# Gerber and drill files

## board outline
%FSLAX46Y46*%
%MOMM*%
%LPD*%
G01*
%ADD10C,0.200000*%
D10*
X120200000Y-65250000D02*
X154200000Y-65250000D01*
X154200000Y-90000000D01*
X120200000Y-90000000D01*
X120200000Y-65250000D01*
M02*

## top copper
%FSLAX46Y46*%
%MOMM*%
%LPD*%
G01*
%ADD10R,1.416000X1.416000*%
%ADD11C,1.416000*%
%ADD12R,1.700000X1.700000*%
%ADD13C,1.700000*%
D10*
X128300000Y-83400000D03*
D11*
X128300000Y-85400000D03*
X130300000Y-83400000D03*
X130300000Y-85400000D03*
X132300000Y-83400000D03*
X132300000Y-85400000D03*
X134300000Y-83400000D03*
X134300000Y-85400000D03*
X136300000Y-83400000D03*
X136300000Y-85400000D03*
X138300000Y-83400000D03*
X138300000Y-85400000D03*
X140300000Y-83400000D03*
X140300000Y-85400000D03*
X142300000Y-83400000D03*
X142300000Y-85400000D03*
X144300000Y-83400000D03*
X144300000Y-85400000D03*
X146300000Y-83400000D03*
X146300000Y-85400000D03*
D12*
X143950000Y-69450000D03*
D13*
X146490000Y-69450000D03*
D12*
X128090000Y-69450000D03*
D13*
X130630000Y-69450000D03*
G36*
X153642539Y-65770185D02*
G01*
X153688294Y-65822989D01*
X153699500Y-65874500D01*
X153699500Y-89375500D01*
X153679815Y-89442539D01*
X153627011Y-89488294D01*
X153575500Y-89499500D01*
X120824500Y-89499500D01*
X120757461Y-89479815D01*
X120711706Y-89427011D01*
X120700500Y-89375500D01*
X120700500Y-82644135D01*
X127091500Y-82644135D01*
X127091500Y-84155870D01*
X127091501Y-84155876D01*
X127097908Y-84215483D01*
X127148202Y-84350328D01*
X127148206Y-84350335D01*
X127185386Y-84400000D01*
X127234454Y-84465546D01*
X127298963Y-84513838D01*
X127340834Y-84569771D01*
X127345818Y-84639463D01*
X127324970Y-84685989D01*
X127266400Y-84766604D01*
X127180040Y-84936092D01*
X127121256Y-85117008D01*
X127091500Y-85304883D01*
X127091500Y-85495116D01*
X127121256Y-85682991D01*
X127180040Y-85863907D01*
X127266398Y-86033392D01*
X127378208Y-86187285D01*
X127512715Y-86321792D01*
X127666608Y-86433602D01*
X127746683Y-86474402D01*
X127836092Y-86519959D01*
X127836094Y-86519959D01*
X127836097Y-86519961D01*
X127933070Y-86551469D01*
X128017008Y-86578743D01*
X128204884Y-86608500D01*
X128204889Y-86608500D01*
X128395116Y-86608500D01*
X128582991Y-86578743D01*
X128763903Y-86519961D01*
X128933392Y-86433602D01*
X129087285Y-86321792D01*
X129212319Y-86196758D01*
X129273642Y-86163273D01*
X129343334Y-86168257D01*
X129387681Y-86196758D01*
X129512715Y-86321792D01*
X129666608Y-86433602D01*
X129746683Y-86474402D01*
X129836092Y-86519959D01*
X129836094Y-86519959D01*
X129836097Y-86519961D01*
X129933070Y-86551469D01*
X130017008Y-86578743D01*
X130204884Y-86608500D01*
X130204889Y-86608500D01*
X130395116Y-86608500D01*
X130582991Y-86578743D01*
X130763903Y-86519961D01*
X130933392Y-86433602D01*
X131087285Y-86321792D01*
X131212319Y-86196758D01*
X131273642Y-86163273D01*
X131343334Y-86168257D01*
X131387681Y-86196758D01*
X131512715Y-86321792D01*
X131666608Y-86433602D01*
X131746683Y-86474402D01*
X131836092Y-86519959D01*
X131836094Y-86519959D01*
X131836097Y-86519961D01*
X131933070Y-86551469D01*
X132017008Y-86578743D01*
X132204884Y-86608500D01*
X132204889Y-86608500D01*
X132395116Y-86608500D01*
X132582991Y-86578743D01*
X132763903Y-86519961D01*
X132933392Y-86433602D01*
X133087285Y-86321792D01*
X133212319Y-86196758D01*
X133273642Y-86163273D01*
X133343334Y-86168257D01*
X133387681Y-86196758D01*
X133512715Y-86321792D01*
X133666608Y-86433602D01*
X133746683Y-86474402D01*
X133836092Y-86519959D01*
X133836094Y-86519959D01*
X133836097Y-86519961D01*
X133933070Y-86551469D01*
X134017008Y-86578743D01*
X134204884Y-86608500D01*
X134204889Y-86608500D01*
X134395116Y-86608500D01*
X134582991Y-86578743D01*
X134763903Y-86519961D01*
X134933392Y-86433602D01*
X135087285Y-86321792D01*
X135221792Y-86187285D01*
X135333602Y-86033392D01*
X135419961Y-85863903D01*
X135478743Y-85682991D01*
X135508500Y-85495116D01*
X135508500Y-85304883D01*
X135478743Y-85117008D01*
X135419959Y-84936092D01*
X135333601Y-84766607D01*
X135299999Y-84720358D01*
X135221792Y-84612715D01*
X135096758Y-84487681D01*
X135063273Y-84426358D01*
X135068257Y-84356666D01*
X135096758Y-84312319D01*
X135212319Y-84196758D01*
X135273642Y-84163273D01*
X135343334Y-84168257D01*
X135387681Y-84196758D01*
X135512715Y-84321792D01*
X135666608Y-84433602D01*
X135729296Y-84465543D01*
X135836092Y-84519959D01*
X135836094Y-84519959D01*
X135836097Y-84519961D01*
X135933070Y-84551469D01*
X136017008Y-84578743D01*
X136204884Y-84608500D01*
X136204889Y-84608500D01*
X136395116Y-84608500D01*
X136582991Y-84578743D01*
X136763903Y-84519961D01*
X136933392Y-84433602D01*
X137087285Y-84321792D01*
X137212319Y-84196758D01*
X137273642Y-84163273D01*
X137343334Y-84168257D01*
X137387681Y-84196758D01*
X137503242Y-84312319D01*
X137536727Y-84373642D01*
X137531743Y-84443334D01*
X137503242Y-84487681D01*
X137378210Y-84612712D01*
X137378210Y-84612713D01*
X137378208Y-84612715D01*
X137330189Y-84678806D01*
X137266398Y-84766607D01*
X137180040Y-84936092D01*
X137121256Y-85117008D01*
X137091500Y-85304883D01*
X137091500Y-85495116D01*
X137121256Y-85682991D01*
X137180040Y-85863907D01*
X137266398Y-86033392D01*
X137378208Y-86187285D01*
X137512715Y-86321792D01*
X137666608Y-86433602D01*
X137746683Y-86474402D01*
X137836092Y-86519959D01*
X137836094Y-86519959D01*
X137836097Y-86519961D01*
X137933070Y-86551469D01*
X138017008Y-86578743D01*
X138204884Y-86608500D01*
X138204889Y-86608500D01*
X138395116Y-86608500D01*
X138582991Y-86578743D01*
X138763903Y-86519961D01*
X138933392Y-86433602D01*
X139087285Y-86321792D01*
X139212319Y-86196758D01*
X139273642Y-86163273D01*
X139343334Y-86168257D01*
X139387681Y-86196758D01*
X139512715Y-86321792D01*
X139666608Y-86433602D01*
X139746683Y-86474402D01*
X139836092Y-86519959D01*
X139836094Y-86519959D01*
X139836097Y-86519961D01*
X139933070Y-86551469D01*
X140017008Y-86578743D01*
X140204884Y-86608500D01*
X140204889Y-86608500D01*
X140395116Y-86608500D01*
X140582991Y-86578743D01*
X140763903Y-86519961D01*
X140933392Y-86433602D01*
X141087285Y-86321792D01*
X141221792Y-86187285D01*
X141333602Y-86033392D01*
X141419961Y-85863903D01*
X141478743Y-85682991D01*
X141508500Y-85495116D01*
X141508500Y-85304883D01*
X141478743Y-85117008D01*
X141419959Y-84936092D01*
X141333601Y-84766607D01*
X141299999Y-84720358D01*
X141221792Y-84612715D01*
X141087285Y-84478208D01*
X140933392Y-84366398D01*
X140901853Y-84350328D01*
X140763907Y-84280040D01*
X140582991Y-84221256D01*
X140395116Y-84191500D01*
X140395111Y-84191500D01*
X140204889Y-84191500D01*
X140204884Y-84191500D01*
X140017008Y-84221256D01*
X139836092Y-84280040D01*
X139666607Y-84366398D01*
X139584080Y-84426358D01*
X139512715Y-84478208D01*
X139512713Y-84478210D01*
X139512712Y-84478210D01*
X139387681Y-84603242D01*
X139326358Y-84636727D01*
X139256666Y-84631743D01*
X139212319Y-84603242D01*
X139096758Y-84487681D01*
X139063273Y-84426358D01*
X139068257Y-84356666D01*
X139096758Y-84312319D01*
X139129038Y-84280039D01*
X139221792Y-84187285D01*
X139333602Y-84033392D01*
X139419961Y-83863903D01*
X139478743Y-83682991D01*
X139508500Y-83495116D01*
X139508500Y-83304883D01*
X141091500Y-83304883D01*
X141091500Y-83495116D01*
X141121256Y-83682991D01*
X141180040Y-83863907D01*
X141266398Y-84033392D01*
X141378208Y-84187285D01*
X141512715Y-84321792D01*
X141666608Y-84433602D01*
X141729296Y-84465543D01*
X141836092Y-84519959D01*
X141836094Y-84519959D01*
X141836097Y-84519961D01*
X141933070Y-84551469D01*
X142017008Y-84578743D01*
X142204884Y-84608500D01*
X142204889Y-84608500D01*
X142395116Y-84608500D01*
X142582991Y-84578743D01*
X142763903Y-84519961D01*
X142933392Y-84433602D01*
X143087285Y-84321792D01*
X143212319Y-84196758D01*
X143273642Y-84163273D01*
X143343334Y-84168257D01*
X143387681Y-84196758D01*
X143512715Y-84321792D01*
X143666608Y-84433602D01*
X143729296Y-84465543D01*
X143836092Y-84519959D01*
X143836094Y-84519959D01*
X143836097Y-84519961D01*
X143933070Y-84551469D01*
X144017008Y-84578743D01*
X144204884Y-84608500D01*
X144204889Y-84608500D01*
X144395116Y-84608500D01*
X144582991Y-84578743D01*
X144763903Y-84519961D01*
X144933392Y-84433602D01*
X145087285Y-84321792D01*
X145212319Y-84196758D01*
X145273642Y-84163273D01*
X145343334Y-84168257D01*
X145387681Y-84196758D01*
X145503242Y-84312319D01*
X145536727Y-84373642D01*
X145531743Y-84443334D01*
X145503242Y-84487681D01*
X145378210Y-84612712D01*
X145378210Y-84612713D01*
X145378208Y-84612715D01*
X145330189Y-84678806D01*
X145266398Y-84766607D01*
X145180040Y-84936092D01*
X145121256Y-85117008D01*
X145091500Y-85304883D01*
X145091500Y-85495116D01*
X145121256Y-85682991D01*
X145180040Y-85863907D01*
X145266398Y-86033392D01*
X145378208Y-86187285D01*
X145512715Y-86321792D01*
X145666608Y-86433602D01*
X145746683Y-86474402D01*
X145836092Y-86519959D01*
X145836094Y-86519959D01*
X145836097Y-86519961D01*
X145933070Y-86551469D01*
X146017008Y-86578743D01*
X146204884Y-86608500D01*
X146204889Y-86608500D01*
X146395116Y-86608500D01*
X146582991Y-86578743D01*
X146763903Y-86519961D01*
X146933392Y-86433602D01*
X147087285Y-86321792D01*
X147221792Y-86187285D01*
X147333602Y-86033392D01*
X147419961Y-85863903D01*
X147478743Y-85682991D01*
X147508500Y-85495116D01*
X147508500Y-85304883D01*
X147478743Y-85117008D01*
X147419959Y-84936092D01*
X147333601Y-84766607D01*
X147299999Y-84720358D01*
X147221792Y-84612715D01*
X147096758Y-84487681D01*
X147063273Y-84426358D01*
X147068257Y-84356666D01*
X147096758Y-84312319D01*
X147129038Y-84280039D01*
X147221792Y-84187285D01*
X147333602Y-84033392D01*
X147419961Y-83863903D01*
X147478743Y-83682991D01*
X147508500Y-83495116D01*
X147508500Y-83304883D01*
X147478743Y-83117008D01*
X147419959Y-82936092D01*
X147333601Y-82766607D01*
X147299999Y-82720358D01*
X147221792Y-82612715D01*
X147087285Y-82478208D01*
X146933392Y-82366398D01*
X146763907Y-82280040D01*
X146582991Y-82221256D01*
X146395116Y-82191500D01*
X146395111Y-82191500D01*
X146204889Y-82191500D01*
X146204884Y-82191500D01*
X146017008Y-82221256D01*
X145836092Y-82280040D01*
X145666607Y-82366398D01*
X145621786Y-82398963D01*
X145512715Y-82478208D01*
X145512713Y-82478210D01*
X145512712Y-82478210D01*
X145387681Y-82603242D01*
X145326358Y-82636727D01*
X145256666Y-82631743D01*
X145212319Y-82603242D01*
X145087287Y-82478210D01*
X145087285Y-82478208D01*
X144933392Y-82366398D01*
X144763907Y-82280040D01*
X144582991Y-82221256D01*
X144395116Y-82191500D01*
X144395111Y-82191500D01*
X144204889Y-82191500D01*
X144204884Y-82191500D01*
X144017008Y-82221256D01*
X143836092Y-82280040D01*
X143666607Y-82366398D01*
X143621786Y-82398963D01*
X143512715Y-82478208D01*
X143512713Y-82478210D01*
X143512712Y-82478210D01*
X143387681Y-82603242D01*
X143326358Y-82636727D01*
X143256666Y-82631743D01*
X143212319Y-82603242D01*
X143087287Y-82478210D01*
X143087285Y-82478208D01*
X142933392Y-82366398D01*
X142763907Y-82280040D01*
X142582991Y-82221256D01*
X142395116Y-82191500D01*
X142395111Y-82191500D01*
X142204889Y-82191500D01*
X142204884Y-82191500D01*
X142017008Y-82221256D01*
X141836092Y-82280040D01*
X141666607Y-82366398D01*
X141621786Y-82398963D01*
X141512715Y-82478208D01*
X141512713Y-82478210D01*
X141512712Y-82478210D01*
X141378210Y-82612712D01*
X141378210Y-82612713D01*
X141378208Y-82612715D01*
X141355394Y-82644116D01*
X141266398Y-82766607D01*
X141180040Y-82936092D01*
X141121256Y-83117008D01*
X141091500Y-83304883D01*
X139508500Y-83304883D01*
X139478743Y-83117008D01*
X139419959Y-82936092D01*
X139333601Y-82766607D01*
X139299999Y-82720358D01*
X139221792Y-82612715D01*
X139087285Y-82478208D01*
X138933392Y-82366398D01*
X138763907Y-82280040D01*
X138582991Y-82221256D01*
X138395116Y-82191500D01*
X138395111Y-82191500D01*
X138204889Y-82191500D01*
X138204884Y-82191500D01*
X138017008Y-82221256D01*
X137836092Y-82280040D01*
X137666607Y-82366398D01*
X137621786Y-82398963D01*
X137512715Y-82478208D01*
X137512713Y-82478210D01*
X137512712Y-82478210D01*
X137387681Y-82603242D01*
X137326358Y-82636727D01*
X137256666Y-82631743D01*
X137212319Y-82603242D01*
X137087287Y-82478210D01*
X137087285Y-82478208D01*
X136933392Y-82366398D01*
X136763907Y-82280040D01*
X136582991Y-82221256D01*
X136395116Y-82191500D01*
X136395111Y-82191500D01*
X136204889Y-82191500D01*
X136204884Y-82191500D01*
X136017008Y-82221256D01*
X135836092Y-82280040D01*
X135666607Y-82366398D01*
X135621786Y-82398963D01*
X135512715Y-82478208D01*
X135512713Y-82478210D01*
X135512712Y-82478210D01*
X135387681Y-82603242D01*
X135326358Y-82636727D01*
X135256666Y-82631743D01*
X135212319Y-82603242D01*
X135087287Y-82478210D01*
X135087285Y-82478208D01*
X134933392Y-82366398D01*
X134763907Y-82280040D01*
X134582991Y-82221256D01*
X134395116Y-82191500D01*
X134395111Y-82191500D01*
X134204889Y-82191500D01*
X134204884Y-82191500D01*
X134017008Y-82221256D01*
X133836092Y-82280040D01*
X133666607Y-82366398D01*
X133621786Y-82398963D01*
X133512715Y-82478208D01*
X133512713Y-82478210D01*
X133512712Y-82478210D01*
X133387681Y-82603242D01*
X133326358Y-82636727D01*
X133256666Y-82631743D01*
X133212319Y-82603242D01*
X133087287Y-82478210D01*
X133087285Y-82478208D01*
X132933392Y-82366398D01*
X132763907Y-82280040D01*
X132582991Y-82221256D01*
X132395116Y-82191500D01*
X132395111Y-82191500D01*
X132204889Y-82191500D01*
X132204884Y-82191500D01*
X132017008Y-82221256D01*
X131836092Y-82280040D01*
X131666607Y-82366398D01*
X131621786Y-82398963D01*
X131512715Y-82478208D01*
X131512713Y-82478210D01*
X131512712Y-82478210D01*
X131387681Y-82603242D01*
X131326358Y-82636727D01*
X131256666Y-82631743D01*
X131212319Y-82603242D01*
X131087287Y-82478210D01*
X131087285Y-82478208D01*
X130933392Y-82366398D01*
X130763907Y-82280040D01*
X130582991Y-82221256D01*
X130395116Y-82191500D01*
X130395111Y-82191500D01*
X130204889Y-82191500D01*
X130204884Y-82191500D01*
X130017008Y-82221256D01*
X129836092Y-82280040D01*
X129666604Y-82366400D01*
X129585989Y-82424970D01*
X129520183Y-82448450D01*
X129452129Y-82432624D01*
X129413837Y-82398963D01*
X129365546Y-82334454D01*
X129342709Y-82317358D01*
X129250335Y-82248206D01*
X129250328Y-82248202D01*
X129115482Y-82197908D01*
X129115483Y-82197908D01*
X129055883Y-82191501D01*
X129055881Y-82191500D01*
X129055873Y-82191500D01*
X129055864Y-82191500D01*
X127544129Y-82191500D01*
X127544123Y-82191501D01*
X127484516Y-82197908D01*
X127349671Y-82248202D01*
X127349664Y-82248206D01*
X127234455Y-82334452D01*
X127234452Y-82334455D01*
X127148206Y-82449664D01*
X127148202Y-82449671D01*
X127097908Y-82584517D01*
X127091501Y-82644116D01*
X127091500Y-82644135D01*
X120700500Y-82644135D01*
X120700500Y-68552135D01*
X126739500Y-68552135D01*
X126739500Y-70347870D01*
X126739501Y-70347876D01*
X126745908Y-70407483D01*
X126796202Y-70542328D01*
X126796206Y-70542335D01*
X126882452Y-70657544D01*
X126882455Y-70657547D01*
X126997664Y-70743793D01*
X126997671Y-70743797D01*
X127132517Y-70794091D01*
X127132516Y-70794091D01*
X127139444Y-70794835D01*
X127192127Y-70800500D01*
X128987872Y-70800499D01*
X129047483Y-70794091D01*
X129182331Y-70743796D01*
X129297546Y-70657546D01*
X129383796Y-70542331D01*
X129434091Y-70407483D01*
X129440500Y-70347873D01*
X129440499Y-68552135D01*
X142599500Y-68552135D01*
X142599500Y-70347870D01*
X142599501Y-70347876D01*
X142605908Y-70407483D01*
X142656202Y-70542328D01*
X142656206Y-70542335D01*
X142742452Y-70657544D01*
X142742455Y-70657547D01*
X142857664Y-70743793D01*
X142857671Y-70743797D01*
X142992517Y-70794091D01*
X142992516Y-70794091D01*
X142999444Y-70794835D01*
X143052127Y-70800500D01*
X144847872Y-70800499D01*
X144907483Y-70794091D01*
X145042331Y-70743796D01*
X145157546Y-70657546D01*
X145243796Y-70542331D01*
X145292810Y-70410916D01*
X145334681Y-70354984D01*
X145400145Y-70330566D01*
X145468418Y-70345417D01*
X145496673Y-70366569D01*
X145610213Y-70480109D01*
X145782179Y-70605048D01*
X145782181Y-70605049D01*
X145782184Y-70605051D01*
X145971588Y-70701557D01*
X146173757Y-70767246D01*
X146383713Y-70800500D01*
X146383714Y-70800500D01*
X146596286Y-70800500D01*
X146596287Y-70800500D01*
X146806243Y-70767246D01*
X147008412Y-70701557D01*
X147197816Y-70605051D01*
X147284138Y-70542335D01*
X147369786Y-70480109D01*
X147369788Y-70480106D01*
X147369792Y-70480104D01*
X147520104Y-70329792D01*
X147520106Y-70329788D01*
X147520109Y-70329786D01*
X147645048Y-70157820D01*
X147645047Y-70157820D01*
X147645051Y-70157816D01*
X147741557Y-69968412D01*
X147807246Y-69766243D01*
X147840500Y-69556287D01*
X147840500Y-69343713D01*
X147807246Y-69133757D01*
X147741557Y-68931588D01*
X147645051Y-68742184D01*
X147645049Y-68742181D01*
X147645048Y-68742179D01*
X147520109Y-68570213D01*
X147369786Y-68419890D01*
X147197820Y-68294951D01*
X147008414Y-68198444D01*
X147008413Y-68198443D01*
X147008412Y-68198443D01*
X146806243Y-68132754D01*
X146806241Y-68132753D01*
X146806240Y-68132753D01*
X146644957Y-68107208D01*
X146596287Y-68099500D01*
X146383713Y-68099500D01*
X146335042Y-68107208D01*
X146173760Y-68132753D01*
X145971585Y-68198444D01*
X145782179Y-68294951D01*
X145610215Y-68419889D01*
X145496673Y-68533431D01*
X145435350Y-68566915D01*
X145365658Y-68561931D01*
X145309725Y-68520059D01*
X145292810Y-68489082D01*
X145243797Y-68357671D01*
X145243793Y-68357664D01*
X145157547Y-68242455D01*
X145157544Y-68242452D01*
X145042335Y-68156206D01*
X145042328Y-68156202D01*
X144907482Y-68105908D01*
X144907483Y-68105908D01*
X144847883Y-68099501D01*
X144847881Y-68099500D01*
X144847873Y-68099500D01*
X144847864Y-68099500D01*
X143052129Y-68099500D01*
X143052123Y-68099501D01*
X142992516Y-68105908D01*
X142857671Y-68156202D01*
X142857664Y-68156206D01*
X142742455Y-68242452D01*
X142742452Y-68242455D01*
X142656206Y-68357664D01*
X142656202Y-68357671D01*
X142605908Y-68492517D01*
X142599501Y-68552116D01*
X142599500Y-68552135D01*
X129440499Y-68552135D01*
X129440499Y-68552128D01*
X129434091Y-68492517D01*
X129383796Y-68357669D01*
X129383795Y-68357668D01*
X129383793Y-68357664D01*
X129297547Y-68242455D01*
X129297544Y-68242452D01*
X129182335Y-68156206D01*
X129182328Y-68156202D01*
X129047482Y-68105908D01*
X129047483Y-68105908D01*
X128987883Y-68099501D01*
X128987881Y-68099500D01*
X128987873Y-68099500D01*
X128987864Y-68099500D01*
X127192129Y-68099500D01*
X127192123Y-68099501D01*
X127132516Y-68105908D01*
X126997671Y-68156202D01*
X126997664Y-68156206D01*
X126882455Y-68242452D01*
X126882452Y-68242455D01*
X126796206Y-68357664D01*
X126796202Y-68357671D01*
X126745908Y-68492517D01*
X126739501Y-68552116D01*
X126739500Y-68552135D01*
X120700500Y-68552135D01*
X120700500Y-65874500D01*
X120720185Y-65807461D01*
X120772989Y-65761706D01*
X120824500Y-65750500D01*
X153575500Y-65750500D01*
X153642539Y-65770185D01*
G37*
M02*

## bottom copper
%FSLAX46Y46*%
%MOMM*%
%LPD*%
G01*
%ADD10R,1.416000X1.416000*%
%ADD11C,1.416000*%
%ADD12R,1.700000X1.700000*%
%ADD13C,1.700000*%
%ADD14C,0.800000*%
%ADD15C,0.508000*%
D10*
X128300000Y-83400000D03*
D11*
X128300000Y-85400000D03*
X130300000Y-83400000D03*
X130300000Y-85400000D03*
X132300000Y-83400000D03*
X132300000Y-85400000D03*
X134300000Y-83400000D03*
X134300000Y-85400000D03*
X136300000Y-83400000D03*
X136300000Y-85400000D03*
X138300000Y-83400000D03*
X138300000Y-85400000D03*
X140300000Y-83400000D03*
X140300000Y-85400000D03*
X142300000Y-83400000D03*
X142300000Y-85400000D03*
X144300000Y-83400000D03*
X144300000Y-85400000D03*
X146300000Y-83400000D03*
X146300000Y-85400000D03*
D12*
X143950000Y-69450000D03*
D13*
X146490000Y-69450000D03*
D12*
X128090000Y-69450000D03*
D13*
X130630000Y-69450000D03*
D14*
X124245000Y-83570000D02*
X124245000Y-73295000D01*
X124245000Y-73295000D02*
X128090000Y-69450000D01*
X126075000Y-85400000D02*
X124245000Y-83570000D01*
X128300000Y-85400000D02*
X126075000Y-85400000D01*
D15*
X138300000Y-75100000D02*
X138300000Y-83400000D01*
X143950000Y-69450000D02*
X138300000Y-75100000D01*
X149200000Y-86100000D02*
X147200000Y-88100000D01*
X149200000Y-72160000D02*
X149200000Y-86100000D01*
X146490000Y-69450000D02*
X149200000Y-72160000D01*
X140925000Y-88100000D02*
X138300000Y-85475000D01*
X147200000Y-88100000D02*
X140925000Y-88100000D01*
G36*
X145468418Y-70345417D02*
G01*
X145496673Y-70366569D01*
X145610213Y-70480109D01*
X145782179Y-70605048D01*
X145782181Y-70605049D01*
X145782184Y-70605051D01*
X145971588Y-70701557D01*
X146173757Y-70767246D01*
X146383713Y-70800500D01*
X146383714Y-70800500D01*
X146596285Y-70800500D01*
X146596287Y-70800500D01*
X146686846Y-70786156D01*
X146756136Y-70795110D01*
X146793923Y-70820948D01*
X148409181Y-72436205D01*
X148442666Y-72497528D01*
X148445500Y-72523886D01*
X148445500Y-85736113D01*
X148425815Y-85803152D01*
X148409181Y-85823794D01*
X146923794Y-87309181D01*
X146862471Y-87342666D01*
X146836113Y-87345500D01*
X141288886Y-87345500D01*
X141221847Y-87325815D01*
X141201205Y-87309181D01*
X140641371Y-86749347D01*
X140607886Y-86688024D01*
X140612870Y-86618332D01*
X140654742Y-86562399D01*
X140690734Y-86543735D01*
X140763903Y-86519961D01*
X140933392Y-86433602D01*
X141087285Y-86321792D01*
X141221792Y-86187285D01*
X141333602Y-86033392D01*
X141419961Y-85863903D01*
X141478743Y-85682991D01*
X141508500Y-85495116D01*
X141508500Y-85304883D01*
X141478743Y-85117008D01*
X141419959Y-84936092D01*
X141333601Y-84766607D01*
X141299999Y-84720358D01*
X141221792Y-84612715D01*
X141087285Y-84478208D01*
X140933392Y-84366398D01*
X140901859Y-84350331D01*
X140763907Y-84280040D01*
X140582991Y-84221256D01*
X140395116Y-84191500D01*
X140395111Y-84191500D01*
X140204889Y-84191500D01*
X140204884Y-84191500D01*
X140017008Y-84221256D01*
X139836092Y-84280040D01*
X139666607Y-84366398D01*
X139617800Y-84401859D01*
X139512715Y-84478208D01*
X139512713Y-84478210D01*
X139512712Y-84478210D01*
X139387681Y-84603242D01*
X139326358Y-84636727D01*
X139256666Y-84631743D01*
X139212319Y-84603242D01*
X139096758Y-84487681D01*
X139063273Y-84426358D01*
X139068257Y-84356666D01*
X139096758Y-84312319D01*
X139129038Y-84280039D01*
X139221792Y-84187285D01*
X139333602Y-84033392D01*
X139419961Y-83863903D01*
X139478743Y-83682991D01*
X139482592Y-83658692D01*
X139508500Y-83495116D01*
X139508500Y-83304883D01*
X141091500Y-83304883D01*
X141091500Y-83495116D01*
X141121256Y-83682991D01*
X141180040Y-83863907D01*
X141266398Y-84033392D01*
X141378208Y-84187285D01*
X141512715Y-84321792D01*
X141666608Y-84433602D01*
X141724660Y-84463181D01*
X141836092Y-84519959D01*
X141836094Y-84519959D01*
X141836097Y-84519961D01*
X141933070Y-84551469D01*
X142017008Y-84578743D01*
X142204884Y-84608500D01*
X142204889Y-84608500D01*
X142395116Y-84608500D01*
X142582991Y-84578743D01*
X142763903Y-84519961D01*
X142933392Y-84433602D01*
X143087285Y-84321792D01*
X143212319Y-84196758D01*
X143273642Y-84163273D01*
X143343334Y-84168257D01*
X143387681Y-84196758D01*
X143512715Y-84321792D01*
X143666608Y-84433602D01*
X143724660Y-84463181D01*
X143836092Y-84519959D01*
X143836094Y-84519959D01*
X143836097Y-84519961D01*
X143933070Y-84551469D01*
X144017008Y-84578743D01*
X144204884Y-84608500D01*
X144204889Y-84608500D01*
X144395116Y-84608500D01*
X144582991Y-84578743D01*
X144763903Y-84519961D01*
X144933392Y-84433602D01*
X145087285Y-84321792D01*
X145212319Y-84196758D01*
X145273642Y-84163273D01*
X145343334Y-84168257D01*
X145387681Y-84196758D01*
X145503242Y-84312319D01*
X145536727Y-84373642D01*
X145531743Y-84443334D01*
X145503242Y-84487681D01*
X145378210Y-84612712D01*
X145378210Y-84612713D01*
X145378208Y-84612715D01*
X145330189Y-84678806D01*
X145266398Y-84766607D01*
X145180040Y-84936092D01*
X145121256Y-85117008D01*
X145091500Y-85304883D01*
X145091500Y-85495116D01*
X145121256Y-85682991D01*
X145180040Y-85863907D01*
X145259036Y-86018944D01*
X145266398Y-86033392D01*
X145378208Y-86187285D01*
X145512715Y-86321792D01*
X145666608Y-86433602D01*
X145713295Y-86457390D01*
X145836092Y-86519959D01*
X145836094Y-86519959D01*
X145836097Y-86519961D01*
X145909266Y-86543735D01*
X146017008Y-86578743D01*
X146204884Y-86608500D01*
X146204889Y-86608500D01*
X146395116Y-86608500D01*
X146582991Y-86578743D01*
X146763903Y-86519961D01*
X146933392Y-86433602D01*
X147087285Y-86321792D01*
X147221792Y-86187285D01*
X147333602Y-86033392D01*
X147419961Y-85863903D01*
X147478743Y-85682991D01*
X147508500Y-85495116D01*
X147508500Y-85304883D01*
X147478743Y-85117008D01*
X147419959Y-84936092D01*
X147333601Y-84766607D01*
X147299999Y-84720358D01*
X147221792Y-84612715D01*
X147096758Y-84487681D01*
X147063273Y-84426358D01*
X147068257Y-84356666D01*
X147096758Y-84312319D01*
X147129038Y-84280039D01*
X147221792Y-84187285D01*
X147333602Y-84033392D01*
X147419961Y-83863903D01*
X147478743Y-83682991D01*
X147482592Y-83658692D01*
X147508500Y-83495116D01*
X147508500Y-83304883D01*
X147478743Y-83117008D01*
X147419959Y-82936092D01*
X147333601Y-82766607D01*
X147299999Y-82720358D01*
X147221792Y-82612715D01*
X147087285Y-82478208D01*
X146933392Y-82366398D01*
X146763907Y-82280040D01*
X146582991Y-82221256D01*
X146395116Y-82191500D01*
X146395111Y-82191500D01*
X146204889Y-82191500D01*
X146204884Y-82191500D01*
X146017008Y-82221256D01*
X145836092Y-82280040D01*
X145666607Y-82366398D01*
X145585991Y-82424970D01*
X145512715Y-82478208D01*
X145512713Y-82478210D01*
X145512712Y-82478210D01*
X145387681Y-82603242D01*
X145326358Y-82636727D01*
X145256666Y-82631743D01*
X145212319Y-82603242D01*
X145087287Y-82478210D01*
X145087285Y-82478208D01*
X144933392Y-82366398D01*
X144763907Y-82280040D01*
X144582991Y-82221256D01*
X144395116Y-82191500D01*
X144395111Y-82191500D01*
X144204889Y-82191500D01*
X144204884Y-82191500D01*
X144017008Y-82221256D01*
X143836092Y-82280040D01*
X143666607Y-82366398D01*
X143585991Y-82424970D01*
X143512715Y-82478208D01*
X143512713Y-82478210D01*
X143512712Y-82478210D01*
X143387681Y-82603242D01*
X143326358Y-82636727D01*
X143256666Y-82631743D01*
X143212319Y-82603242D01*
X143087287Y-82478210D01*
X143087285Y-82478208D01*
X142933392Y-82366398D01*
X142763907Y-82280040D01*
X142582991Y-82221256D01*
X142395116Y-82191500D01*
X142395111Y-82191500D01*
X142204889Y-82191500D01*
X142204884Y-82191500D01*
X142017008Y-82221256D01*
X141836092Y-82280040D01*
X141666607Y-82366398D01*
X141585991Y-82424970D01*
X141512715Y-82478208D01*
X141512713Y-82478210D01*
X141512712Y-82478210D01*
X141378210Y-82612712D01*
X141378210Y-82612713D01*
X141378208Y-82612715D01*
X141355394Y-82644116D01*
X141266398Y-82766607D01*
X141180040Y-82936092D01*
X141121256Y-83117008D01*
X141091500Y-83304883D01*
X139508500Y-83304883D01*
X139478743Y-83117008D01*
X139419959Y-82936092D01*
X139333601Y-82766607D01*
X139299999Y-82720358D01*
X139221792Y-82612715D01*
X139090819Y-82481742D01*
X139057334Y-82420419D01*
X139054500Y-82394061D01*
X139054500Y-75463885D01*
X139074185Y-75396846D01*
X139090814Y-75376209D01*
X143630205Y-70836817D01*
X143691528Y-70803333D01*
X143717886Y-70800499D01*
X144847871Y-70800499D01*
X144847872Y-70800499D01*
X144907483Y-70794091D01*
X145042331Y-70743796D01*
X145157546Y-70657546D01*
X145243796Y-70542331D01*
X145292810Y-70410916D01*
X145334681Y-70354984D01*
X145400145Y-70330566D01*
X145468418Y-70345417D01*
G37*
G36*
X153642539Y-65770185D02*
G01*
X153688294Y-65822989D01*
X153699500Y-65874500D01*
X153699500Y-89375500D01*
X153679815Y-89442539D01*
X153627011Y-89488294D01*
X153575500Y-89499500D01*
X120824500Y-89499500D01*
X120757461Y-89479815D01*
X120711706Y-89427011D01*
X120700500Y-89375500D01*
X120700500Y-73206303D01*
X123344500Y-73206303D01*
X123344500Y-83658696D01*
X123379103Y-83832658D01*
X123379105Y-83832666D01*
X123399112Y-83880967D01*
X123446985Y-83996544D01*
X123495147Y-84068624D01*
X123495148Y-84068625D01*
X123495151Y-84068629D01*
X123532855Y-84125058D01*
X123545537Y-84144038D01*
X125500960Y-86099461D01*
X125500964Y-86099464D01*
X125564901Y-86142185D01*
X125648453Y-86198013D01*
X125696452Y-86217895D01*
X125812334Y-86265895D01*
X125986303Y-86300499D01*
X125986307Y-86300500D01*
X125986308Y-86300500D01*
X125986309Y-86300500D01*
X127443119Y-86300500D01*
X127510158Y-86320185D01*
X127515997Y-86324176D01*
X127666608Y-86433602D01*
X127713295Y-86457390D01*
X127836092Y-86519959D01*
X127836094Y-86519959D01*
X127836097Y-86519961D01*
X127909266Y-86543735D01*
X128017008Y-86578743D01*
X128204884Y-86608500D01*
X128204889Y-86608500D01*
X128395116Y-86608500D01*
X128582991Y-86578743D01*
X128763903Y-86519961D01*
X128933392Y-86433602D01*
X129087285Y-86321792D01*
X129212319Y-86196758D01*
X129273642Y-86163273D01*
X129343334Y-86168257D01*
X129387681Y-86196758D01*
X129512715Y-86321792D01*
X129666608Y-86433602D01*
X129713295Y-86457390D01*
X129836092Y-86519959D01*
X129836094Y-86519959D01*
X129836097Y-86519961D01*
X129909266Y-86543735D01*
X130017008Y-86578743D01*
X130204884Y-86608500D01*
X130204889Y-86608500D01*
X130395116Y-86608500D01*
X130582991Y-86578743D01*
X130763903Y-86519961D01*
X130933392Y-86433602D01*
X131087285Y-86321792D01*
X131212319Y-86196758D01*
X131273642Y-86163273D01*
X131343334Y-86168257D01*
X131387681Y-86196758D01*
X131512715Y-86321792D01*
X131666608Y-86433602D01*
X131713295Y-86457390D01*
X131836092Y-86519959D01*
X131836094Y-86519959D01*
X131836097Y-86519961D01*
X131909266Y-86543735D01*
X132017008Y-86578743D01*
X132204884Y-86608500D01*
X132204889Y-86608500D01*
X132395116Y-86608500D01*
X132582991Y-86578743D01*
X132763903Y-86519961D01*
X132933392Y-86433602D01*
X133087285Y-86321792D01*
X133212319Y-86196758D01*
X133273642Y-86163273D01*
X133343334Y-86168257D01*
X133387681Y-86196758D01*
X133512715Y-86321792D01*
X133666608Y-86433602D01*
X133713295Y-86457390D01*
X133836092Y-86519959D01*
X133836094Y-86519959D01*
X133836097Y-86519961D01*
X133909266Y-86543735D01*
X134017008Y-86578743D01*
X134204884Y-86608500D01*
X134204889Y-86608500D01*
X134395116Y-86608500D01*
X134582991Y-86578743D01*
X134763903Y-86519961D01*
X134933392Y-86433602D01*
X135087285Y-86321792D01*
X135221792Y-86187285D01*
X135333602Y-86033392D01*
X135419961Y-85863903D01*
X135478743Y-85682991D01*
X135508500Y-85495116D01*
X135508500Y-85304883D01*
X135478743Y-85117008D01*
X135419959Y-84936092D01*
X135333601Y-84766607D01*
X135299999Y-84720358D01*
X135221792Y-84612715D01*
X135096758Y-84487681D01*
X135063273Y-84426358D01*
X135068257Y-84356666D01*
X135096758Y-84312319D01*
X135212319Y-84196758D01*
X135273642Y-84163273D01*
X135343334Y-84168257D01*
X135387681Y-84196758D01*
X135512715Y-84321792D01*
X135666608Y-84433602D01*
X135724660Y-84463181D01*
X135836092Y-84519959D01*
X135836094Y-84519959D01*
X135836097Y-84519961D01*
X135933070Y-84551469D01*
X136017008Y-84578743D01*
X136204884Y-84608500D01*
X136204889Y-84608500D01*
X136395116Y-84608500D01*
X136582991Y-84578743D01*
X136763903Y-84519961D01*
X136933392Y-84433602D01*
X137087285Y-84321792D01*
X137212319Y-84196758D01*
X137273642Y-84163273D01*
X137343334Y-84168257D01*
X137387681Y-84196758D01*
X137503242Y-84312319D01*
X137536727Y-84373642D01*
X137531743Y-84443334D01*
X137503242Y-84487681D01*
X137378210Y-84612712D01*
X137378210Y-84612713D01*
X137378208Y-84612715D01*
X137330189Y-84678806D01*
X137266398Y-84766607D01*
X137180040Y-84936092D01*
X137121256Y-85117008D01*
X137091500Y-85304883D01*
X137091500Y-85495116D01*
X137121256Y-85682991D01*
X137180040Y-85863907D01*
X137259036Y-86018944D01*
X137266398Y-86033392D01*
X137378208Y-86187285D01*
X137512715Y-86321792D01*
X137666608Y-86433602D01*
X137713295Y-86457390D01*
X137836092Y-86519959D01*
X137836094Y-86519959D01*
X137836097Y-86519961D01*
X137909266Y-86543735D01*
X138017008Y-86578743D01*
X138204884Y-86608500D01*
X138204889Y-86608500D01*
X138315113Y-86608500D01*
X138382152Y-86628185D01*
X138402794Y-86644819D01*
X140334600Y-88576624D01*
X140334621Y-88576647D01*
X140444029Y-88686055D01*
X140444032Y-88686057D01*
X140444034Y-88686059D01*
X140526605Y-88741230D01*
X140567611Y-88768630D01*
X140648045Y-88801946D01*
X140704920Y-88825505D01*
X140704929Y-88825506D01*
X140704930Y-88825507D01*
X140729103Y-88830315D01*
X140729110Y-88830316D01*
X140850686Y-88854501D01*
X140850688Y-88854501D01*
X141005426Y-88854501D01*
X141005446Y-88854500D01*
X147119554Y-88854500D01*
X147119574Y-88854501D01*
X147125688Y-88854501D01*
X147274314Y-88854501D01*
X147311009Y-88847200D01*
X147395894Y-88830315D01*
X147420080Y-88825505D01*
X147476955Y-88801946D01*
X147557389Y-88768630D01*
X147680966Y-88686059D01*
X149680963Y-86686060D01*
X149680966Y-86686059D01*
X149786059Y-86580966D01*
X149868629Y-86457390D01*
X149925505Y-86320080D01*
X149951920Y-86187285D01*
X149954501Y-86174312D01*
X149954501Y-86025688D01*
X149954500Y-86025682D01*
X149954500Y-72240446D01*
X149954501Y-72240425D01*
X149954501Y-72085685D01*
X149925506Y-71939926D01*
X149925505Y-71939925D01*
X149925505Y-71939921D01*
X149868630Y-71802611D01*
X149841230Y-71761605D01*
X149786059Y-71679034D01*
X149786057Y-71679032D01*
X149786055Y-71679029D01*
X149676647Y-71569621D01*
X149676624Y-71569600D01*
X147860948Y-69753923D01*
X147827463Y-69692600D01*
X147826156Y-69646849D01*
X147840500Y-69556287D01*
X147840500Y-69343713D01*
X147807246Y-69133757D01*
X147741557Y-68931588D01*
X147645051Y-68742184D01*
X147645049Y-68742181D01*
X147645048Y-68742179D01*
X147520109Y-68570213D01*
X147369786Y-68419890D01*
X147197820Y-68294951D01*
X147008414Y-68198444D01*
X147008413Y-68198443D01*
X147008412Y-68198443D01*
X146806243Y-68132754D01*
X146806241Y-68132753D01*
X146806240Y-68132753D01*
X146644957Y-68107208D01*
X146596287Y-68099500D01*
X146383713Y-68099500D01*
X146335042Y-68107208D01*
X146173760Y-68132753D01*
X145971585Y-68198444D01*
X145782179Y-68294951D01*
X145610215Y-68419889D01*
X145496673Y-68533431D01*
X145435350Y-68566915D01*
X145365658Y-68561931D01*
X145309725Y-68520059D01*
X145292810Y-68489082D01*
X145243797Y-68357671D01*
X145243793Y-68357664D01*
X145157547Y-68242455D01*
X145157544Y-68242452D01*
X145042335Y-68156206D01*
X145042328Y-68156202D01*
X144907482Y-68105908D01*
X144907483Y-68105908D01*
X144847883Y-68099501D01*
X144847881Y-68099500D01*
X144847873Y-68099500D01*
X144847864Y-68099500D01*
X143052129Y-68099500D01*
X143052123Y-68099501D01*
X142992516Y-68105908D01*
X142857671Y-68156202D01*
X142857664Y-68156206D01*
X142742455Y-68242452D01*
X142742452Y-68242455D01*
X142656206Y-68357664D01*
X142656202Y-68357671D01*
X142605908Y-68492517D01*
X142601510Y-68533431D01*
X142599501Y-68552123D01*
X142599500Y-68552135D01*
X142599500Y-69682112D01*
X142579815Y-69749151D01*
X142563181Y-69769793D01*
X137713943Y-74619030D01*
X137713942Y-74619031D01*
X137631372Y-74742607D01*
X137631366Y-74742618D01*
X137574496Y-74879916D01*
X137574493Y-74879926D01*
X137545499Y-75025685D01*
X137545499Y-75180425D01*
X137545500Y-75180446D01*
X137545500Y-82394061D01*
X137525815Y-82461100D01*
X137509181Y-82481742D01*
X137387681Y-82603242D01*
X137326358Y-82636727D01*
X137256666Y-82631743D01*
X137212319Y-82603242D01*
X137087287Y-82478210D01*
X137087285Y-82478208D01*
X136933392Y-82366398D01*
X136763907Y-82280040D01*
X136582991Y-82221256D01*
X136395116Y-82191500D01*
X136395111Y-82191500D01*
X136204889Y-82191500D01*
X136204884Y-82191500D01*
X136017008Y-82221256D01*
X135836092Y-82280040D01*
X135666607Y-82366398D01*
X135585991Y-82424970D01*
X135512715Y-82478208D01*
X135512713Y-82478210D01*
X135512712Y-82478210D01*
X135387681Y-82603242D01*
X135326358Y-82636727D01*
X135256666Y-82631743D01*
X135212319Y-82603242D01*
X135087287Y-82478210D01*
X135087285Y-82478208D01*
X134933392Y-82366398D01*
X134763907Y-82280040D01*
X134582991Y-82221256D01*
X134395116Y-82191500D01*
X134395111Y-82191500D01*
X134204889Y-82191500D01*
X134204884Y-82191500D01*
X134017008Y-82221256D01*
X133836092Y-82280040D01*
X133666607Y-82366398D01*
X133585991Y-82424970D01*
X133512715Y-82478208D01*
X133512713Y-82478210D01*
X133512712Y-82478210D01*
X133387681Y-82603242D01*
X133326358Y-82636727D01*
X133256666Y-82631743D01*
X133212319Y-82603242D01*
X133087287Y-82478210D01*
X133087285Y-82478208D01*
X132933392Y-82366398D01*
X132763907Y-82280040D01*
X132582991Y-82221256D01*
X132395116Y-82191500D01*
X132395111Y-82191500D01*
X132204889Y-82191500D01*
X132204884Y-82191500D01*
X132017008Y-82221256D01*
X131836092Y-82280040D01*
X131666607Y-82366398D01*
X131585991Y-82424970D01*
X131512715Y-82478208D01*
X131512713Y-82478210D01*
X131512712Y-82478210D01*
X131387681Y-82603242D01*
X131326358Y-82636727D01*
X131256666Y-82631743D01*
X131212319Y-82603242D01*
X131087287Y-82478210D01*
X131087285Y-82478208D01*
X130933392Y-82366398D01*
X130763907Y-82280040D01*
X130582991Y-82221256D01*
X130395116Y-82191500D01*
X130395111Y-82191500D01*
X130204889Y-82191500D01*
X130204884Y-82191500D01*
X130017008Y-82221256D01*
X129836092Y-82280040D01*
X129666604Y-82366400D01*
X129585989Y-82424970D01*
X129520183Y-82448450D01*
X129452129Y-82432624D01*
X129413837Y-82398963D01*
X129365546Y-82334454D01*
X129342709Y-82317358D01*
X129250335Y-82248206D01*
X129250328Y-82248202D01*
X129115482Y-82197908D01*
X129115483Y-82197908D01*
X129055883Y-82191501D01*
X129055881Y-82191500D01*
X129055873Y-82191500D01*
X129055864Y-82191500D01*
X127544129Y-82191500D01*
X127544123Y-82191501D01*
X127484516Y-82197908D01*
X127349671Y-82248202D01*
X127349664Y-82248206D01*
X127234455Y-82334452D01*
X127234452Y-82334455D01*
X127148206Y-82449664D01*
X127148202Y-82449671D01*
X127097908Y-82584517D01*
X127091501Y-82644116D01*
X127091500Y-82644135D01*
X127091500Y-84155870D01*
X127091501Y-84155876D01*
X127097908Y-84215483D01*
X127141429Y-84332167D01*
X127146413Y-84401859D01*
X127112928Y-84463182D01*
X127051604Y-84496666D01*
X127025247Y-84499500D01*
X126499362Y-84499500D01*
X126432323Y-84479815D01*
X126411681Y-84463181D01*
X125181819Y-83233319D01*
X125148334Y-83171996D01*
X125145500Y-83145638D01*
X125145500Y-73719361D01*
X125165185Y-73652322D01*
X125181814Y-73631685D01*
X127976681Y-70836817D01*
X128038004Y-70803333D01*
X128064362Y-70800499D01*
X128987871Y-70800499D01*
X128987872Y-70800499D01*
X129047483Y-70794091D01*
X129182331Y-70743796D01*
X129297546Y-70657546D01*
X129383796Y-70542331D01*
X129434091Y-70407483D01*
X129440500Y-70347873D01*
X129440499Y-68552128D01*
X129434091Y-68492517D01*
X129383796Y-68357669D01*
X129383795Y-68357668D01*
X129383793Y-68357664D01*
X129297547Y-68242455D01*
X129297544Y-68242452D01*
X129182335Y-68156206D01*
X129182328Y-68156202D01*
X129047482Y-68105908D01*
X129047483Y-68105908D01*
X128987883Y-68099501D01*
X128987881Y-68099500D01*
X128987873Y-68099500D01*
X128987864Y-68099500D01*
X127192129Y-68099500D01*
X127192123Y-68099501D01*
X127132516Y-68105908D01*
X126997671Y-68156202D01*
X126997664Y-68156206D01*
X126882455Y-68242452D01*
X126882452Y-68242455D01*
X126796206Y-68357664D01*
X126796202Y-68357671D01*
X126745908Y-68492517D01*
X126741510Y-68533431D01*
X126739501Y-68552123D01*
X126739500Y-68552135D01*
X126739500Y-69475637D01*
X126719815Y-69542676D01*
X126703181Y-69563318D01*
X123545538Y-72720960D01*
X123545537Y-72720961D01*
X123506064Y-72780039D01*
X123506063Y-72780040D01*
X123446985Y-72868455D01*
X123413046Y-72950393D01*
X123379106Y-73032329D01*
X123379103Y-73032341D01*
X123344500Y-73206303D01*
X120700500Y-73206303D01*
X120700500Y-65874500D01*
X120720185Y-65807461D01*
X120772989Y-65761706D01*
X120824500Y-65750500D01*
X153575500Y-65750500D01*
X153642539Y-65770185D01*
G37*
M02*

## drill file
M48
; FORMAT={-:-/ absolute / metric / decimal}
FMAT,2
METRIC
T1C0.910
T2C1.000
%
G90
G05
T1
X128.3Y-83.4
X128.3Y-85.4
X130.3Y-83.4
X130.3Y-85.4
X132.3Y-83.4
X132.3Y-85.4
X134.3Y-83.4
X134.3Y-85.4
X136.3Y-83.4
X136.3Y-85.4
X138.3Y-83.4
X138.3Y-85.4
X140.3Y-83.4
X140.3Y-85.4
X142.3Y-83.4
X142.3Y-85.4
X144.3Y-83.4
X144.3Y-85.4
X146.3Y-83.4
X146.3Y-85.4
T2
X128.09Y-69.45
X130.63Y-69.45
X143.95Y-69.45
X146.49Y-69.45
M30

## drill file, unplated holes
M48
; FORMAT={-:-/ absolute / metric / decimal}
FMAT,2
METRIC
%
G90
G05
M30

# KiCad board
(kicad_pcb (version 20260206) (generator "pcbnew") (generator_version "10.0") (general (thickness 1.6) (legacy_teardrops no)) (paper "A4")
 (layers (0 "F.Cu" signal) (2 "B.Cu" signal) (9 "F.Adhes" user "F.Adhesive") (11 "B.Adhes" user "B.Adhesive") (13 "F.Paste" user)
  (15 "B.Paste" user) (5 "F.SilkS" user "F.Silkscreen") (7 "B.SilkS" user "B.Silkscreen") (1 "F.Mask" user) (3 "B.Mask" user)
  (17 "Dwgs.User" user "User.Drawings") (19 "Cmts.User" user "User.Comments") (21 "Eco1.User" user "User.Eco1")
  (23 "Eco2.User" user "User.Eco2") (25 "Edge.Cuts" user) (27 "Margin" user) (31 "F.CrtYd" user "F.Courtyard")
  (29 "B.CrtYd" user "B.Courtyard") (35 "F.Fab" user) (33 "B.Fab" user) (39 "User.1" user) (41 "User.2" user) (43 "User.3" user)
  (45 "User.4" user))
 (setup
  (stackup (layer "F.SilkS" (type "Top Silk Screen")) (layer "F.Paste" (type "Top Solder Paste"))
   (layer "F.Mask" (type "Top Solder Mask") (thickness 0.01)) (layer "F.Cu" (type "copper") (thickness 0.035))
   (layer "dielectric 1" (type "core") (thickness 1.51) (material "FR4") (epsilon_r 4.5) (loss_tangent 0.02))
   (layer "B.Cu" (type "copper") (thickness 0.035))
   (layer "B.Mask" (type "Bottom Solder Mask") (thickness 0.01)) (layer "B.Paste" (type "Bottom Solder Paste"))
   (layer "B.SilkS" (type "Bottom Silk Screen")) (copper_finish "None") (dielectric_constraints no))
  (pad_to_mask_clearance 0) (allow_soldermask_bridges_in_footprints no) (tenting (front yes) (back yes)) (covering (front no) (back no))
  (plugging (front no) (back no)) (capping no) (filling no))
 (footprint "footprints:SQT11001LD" (layer "F.Cu") (at 128.3 83.4 180)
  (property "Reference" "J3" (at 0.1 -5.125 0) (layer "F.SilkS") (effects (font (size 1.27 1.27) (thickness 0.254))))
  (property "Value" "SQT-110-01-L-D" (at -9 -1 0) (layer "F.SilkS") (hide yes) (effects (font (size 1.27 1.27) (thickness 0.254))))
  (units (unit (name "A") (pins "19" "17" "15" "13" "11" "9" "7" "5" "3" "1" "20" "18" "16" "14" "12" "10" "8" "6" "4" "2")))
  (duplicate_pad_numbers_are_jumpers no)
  (pad "1" thru_hole rect (at 0 0 180) (size 1.416 1.416) (drill 0.91) (layers "*.Cu" "*.Mask") (remove_unused_layers no)
   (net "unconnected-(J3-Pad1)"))
  (pad "2" thru_hole circle (at 0 -2 180) (size 1.416 1.416) (drill 0.91) (layers "*.Cu" "*.Mask") (remove_unused_layers no) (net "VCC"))
  (pad "3" thru_hole circle (at -2 0 180) (size 1.416 1.416) (drill 0.91) (layers "*.Cu" "*.Mask") (remove_unused_layers no)
   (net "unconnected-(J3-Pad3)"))
  (pad "4" thru_hole circle (at -2 -2 180) (size 1.416 1.416) (drill 0.91) (layers "*.Cu" "*.Mask") (remove_unused_layers no)
   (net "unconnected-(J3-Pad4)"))
  (pad "5" thru_hole circle (at -4 0 180) (size 1.416 1.416) (drill 0.91) (layers "*.Cu" "*.Mask") (remove_unused_layers no)
   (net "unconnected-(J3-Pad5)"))
  (pad "6" thru_hole circle (at -4 -2 180) (size 1.416 1.416) (drill 0.91) (layers "*.Cu" "*.Mask") (remove_unused_layers no)
   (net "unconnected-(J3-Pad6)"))
  (pad "7" thru_hole circle (at -6 0 180) (size 1.416 1.416) (drill 0.91) (layers "*.Cu" "*.Mask") (remove_unused_layers no)
   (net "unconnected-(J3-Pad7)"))
  (pad "8" thru_hole circle (at -6 -2 180) (size 1.416 1.416) (drill 0.91) (layers "*.Cu" "*.Mask") (remove_unused_layers no)
   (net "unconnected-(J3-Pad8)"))
  (pad "9" thru_hole circle (at -8 0 180) (size 1.416 1.416) (drill 0.91) (layers "*.Cu" "*.Mask") (remove_unused_layers no)
   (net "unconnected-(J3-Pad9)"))
  (pad "10" thru_hole circle (at -8 -2 180) (size 1.416 1.416) (drill 0.91) (layers "*.Cu" "*.Mask") (remove_unused_layers no)
   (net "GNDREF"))
  (pad "11" thru_hole circle (at -10 0 180) (size 1.416 1.416) (drill 0.91) (layers "*.Cu" "*.Mask") (remove_unused_layers no) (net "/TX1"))
  (pad "12" thru_hole circle (at -10 -2 180) (size 1.416 1.416) (drill 0.91) (layers "*.Cu" "*.Mask") (remove_unused_layers no) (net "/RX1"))
  (pad "13" thru_hole circle (at -12 0 180) (size 1.416 1.416) (drill 0.91) (layers "*.Cu" "*.Mask") (remove_unused_layers no)
   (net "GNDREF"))
  (pad "14" thru_hole circle (at -12 -2 180) (size 1.416 1.416) (drill 0.91) (layers "*.Cu" "*.Mask") (remove_unused_layers no)
   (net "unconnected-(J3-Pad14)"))
  (pad "15" thru_hole circle (at -14 0 180) (size 1.416 1.416) (drill 0.91) (layers "*.Cu" "*.Mask") (remove_unused_layers no)
   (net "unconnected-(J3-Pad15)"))
  (pad "16" thru_hole circle (at -14 -2 180) (size 1.416 1.416) (drill 0.91) (layers "*.Cu" "*.Mask") (remove_unused_layers no)
   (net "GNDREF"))
  (pad "17" thru_hole circle (at -16 0 180) (size 1.416 1.416) (drill 0.91) (layers "*.Cu" "*.Mask") (remove_unused_layers no)
   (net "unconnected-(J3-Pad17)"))
  (pad "18" thru_hole circle (at -16 -2 180) (size 1.416 1.416) (drill 0.91) (layers "*.Cu" "*.Mask") (remove_unused_layers no)
   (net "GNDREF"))
  (pad "19" thru_hole circle (at -18 0 180) (size 1.416 1.416) (drill 0.91) (layers "*.Cu" "*.Mask") (remove_unused_layers no)
   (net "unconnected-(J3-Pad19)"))
  (pad "20" thru_hole circle (at -18 -2 180) (size 1.416 1.416) (drill 0.91) (layers "*.Cu" "*.Mask") (remove_unused_layers no)
   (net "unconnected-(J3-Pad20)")))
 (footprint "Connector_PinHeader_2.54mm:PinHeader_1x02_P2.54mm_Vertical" (layer "F.Cu") (at 143.95 69.45 90)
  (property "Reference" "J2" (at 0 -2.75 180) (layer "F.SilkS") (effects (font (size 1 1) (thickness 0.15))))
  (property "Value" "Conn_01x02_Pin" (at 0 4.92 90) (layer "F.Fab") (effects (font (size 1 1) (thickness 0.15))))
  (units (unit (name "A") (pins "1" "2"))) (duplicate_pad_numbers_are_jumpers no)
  (pad "1" thru_hole rect (at 0 0 90) (size 1.7 1.7) (drill 1) (layers "*.Cu" "*.Mask") (remove_unused_layers no) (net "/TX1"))
  (pad "2" thru_hole circle (at 0 2.54 90) (size 1.7 1.7) (drill 1) (layers "*.Cu" "*.Mask") (remove_unused_layers no) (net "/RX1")))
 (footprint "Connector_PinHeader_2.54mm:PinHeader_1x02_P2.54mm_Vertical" (layer "F.Cu") (at 128.09 69.45 90)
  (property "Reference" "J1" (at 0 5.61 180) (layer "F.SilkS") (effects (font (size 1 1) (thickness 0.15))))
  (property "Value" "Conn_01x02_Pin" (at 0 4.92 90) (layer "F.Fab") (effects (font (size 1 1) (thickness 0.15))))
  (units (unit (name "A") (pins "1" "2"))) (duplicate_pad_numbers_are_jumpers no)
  (pad "1" thru_hole rect (at 0 0 90) (size 1.7 1.7) (drill 1) (layers "*.Cu" "*.Mask") (remove_unused_layers no) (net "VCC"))
  (pad "2" thru_hole circle (at 0 2.54 90) (size 1.7 1.7) (drill 1) (layers "*.Cu" "*.Mask") (remove_unused_layers no) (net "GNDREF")))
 (gr_rect (start 120.2 65.25) (end 154.2 90) (stroke (width 0.2) (type solid)) (fill no) (layer "Edge.Cuts"))
 (segment (start 124.245 83.57) (end 124.245 73.295) (width 0.8) (layer "B.Cu") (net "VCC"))
 (segment (start 124.245 73.295) (end 128.09 69.45) (width 0.8) (layer "B.Cu") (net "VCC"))
 (segment (start 126.075 85.4) (end 124.245 83.57) (width 0.8) (layer "B.Cu") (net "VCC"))
 (segment (start 128.3 85.4) (end 126.075 85.4) (width 0.8) (layer "B.Cu") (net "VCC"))
 (segment (start 138.3 75.1) (end 138.3 83.4) (width 0.508) (layer "B.Cu") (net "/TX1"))
 (segment (start 143.95 69.45) (end 138.3 75.1) (width 0.508) (layer "B.Cu") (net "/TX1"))
 (segment (start 149.2 86.1) (end 147.2 88.1) (width 0.508) (layer "B.Cu") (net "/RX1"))
 (segment (start 149.2 72.16) (end 149.2 86.1) (width 0.508) (layer "B.Cu") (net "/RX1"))
 (segment (start 146.49 69.45) (end 149.2 72.16) (width 0.508) (layer "B.Cu") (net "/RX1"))
 (segment (start 140.925 88.1) (end 138.3 85.475) (width 0.508) (layer "B.Cu") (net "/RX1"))
 (segment (start 147.2 88.1) (end 140.925 88.1) (width 0.508) (layer "B.Cu") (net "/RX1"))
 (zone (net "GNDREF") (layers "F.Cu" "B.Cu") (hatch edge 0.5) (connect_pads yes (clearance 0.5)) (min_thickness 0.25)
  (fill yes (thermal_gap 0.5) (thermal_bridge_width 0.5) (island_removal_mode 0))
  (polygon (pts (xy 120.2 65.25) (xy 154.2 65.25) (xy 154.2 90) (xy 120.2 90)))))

